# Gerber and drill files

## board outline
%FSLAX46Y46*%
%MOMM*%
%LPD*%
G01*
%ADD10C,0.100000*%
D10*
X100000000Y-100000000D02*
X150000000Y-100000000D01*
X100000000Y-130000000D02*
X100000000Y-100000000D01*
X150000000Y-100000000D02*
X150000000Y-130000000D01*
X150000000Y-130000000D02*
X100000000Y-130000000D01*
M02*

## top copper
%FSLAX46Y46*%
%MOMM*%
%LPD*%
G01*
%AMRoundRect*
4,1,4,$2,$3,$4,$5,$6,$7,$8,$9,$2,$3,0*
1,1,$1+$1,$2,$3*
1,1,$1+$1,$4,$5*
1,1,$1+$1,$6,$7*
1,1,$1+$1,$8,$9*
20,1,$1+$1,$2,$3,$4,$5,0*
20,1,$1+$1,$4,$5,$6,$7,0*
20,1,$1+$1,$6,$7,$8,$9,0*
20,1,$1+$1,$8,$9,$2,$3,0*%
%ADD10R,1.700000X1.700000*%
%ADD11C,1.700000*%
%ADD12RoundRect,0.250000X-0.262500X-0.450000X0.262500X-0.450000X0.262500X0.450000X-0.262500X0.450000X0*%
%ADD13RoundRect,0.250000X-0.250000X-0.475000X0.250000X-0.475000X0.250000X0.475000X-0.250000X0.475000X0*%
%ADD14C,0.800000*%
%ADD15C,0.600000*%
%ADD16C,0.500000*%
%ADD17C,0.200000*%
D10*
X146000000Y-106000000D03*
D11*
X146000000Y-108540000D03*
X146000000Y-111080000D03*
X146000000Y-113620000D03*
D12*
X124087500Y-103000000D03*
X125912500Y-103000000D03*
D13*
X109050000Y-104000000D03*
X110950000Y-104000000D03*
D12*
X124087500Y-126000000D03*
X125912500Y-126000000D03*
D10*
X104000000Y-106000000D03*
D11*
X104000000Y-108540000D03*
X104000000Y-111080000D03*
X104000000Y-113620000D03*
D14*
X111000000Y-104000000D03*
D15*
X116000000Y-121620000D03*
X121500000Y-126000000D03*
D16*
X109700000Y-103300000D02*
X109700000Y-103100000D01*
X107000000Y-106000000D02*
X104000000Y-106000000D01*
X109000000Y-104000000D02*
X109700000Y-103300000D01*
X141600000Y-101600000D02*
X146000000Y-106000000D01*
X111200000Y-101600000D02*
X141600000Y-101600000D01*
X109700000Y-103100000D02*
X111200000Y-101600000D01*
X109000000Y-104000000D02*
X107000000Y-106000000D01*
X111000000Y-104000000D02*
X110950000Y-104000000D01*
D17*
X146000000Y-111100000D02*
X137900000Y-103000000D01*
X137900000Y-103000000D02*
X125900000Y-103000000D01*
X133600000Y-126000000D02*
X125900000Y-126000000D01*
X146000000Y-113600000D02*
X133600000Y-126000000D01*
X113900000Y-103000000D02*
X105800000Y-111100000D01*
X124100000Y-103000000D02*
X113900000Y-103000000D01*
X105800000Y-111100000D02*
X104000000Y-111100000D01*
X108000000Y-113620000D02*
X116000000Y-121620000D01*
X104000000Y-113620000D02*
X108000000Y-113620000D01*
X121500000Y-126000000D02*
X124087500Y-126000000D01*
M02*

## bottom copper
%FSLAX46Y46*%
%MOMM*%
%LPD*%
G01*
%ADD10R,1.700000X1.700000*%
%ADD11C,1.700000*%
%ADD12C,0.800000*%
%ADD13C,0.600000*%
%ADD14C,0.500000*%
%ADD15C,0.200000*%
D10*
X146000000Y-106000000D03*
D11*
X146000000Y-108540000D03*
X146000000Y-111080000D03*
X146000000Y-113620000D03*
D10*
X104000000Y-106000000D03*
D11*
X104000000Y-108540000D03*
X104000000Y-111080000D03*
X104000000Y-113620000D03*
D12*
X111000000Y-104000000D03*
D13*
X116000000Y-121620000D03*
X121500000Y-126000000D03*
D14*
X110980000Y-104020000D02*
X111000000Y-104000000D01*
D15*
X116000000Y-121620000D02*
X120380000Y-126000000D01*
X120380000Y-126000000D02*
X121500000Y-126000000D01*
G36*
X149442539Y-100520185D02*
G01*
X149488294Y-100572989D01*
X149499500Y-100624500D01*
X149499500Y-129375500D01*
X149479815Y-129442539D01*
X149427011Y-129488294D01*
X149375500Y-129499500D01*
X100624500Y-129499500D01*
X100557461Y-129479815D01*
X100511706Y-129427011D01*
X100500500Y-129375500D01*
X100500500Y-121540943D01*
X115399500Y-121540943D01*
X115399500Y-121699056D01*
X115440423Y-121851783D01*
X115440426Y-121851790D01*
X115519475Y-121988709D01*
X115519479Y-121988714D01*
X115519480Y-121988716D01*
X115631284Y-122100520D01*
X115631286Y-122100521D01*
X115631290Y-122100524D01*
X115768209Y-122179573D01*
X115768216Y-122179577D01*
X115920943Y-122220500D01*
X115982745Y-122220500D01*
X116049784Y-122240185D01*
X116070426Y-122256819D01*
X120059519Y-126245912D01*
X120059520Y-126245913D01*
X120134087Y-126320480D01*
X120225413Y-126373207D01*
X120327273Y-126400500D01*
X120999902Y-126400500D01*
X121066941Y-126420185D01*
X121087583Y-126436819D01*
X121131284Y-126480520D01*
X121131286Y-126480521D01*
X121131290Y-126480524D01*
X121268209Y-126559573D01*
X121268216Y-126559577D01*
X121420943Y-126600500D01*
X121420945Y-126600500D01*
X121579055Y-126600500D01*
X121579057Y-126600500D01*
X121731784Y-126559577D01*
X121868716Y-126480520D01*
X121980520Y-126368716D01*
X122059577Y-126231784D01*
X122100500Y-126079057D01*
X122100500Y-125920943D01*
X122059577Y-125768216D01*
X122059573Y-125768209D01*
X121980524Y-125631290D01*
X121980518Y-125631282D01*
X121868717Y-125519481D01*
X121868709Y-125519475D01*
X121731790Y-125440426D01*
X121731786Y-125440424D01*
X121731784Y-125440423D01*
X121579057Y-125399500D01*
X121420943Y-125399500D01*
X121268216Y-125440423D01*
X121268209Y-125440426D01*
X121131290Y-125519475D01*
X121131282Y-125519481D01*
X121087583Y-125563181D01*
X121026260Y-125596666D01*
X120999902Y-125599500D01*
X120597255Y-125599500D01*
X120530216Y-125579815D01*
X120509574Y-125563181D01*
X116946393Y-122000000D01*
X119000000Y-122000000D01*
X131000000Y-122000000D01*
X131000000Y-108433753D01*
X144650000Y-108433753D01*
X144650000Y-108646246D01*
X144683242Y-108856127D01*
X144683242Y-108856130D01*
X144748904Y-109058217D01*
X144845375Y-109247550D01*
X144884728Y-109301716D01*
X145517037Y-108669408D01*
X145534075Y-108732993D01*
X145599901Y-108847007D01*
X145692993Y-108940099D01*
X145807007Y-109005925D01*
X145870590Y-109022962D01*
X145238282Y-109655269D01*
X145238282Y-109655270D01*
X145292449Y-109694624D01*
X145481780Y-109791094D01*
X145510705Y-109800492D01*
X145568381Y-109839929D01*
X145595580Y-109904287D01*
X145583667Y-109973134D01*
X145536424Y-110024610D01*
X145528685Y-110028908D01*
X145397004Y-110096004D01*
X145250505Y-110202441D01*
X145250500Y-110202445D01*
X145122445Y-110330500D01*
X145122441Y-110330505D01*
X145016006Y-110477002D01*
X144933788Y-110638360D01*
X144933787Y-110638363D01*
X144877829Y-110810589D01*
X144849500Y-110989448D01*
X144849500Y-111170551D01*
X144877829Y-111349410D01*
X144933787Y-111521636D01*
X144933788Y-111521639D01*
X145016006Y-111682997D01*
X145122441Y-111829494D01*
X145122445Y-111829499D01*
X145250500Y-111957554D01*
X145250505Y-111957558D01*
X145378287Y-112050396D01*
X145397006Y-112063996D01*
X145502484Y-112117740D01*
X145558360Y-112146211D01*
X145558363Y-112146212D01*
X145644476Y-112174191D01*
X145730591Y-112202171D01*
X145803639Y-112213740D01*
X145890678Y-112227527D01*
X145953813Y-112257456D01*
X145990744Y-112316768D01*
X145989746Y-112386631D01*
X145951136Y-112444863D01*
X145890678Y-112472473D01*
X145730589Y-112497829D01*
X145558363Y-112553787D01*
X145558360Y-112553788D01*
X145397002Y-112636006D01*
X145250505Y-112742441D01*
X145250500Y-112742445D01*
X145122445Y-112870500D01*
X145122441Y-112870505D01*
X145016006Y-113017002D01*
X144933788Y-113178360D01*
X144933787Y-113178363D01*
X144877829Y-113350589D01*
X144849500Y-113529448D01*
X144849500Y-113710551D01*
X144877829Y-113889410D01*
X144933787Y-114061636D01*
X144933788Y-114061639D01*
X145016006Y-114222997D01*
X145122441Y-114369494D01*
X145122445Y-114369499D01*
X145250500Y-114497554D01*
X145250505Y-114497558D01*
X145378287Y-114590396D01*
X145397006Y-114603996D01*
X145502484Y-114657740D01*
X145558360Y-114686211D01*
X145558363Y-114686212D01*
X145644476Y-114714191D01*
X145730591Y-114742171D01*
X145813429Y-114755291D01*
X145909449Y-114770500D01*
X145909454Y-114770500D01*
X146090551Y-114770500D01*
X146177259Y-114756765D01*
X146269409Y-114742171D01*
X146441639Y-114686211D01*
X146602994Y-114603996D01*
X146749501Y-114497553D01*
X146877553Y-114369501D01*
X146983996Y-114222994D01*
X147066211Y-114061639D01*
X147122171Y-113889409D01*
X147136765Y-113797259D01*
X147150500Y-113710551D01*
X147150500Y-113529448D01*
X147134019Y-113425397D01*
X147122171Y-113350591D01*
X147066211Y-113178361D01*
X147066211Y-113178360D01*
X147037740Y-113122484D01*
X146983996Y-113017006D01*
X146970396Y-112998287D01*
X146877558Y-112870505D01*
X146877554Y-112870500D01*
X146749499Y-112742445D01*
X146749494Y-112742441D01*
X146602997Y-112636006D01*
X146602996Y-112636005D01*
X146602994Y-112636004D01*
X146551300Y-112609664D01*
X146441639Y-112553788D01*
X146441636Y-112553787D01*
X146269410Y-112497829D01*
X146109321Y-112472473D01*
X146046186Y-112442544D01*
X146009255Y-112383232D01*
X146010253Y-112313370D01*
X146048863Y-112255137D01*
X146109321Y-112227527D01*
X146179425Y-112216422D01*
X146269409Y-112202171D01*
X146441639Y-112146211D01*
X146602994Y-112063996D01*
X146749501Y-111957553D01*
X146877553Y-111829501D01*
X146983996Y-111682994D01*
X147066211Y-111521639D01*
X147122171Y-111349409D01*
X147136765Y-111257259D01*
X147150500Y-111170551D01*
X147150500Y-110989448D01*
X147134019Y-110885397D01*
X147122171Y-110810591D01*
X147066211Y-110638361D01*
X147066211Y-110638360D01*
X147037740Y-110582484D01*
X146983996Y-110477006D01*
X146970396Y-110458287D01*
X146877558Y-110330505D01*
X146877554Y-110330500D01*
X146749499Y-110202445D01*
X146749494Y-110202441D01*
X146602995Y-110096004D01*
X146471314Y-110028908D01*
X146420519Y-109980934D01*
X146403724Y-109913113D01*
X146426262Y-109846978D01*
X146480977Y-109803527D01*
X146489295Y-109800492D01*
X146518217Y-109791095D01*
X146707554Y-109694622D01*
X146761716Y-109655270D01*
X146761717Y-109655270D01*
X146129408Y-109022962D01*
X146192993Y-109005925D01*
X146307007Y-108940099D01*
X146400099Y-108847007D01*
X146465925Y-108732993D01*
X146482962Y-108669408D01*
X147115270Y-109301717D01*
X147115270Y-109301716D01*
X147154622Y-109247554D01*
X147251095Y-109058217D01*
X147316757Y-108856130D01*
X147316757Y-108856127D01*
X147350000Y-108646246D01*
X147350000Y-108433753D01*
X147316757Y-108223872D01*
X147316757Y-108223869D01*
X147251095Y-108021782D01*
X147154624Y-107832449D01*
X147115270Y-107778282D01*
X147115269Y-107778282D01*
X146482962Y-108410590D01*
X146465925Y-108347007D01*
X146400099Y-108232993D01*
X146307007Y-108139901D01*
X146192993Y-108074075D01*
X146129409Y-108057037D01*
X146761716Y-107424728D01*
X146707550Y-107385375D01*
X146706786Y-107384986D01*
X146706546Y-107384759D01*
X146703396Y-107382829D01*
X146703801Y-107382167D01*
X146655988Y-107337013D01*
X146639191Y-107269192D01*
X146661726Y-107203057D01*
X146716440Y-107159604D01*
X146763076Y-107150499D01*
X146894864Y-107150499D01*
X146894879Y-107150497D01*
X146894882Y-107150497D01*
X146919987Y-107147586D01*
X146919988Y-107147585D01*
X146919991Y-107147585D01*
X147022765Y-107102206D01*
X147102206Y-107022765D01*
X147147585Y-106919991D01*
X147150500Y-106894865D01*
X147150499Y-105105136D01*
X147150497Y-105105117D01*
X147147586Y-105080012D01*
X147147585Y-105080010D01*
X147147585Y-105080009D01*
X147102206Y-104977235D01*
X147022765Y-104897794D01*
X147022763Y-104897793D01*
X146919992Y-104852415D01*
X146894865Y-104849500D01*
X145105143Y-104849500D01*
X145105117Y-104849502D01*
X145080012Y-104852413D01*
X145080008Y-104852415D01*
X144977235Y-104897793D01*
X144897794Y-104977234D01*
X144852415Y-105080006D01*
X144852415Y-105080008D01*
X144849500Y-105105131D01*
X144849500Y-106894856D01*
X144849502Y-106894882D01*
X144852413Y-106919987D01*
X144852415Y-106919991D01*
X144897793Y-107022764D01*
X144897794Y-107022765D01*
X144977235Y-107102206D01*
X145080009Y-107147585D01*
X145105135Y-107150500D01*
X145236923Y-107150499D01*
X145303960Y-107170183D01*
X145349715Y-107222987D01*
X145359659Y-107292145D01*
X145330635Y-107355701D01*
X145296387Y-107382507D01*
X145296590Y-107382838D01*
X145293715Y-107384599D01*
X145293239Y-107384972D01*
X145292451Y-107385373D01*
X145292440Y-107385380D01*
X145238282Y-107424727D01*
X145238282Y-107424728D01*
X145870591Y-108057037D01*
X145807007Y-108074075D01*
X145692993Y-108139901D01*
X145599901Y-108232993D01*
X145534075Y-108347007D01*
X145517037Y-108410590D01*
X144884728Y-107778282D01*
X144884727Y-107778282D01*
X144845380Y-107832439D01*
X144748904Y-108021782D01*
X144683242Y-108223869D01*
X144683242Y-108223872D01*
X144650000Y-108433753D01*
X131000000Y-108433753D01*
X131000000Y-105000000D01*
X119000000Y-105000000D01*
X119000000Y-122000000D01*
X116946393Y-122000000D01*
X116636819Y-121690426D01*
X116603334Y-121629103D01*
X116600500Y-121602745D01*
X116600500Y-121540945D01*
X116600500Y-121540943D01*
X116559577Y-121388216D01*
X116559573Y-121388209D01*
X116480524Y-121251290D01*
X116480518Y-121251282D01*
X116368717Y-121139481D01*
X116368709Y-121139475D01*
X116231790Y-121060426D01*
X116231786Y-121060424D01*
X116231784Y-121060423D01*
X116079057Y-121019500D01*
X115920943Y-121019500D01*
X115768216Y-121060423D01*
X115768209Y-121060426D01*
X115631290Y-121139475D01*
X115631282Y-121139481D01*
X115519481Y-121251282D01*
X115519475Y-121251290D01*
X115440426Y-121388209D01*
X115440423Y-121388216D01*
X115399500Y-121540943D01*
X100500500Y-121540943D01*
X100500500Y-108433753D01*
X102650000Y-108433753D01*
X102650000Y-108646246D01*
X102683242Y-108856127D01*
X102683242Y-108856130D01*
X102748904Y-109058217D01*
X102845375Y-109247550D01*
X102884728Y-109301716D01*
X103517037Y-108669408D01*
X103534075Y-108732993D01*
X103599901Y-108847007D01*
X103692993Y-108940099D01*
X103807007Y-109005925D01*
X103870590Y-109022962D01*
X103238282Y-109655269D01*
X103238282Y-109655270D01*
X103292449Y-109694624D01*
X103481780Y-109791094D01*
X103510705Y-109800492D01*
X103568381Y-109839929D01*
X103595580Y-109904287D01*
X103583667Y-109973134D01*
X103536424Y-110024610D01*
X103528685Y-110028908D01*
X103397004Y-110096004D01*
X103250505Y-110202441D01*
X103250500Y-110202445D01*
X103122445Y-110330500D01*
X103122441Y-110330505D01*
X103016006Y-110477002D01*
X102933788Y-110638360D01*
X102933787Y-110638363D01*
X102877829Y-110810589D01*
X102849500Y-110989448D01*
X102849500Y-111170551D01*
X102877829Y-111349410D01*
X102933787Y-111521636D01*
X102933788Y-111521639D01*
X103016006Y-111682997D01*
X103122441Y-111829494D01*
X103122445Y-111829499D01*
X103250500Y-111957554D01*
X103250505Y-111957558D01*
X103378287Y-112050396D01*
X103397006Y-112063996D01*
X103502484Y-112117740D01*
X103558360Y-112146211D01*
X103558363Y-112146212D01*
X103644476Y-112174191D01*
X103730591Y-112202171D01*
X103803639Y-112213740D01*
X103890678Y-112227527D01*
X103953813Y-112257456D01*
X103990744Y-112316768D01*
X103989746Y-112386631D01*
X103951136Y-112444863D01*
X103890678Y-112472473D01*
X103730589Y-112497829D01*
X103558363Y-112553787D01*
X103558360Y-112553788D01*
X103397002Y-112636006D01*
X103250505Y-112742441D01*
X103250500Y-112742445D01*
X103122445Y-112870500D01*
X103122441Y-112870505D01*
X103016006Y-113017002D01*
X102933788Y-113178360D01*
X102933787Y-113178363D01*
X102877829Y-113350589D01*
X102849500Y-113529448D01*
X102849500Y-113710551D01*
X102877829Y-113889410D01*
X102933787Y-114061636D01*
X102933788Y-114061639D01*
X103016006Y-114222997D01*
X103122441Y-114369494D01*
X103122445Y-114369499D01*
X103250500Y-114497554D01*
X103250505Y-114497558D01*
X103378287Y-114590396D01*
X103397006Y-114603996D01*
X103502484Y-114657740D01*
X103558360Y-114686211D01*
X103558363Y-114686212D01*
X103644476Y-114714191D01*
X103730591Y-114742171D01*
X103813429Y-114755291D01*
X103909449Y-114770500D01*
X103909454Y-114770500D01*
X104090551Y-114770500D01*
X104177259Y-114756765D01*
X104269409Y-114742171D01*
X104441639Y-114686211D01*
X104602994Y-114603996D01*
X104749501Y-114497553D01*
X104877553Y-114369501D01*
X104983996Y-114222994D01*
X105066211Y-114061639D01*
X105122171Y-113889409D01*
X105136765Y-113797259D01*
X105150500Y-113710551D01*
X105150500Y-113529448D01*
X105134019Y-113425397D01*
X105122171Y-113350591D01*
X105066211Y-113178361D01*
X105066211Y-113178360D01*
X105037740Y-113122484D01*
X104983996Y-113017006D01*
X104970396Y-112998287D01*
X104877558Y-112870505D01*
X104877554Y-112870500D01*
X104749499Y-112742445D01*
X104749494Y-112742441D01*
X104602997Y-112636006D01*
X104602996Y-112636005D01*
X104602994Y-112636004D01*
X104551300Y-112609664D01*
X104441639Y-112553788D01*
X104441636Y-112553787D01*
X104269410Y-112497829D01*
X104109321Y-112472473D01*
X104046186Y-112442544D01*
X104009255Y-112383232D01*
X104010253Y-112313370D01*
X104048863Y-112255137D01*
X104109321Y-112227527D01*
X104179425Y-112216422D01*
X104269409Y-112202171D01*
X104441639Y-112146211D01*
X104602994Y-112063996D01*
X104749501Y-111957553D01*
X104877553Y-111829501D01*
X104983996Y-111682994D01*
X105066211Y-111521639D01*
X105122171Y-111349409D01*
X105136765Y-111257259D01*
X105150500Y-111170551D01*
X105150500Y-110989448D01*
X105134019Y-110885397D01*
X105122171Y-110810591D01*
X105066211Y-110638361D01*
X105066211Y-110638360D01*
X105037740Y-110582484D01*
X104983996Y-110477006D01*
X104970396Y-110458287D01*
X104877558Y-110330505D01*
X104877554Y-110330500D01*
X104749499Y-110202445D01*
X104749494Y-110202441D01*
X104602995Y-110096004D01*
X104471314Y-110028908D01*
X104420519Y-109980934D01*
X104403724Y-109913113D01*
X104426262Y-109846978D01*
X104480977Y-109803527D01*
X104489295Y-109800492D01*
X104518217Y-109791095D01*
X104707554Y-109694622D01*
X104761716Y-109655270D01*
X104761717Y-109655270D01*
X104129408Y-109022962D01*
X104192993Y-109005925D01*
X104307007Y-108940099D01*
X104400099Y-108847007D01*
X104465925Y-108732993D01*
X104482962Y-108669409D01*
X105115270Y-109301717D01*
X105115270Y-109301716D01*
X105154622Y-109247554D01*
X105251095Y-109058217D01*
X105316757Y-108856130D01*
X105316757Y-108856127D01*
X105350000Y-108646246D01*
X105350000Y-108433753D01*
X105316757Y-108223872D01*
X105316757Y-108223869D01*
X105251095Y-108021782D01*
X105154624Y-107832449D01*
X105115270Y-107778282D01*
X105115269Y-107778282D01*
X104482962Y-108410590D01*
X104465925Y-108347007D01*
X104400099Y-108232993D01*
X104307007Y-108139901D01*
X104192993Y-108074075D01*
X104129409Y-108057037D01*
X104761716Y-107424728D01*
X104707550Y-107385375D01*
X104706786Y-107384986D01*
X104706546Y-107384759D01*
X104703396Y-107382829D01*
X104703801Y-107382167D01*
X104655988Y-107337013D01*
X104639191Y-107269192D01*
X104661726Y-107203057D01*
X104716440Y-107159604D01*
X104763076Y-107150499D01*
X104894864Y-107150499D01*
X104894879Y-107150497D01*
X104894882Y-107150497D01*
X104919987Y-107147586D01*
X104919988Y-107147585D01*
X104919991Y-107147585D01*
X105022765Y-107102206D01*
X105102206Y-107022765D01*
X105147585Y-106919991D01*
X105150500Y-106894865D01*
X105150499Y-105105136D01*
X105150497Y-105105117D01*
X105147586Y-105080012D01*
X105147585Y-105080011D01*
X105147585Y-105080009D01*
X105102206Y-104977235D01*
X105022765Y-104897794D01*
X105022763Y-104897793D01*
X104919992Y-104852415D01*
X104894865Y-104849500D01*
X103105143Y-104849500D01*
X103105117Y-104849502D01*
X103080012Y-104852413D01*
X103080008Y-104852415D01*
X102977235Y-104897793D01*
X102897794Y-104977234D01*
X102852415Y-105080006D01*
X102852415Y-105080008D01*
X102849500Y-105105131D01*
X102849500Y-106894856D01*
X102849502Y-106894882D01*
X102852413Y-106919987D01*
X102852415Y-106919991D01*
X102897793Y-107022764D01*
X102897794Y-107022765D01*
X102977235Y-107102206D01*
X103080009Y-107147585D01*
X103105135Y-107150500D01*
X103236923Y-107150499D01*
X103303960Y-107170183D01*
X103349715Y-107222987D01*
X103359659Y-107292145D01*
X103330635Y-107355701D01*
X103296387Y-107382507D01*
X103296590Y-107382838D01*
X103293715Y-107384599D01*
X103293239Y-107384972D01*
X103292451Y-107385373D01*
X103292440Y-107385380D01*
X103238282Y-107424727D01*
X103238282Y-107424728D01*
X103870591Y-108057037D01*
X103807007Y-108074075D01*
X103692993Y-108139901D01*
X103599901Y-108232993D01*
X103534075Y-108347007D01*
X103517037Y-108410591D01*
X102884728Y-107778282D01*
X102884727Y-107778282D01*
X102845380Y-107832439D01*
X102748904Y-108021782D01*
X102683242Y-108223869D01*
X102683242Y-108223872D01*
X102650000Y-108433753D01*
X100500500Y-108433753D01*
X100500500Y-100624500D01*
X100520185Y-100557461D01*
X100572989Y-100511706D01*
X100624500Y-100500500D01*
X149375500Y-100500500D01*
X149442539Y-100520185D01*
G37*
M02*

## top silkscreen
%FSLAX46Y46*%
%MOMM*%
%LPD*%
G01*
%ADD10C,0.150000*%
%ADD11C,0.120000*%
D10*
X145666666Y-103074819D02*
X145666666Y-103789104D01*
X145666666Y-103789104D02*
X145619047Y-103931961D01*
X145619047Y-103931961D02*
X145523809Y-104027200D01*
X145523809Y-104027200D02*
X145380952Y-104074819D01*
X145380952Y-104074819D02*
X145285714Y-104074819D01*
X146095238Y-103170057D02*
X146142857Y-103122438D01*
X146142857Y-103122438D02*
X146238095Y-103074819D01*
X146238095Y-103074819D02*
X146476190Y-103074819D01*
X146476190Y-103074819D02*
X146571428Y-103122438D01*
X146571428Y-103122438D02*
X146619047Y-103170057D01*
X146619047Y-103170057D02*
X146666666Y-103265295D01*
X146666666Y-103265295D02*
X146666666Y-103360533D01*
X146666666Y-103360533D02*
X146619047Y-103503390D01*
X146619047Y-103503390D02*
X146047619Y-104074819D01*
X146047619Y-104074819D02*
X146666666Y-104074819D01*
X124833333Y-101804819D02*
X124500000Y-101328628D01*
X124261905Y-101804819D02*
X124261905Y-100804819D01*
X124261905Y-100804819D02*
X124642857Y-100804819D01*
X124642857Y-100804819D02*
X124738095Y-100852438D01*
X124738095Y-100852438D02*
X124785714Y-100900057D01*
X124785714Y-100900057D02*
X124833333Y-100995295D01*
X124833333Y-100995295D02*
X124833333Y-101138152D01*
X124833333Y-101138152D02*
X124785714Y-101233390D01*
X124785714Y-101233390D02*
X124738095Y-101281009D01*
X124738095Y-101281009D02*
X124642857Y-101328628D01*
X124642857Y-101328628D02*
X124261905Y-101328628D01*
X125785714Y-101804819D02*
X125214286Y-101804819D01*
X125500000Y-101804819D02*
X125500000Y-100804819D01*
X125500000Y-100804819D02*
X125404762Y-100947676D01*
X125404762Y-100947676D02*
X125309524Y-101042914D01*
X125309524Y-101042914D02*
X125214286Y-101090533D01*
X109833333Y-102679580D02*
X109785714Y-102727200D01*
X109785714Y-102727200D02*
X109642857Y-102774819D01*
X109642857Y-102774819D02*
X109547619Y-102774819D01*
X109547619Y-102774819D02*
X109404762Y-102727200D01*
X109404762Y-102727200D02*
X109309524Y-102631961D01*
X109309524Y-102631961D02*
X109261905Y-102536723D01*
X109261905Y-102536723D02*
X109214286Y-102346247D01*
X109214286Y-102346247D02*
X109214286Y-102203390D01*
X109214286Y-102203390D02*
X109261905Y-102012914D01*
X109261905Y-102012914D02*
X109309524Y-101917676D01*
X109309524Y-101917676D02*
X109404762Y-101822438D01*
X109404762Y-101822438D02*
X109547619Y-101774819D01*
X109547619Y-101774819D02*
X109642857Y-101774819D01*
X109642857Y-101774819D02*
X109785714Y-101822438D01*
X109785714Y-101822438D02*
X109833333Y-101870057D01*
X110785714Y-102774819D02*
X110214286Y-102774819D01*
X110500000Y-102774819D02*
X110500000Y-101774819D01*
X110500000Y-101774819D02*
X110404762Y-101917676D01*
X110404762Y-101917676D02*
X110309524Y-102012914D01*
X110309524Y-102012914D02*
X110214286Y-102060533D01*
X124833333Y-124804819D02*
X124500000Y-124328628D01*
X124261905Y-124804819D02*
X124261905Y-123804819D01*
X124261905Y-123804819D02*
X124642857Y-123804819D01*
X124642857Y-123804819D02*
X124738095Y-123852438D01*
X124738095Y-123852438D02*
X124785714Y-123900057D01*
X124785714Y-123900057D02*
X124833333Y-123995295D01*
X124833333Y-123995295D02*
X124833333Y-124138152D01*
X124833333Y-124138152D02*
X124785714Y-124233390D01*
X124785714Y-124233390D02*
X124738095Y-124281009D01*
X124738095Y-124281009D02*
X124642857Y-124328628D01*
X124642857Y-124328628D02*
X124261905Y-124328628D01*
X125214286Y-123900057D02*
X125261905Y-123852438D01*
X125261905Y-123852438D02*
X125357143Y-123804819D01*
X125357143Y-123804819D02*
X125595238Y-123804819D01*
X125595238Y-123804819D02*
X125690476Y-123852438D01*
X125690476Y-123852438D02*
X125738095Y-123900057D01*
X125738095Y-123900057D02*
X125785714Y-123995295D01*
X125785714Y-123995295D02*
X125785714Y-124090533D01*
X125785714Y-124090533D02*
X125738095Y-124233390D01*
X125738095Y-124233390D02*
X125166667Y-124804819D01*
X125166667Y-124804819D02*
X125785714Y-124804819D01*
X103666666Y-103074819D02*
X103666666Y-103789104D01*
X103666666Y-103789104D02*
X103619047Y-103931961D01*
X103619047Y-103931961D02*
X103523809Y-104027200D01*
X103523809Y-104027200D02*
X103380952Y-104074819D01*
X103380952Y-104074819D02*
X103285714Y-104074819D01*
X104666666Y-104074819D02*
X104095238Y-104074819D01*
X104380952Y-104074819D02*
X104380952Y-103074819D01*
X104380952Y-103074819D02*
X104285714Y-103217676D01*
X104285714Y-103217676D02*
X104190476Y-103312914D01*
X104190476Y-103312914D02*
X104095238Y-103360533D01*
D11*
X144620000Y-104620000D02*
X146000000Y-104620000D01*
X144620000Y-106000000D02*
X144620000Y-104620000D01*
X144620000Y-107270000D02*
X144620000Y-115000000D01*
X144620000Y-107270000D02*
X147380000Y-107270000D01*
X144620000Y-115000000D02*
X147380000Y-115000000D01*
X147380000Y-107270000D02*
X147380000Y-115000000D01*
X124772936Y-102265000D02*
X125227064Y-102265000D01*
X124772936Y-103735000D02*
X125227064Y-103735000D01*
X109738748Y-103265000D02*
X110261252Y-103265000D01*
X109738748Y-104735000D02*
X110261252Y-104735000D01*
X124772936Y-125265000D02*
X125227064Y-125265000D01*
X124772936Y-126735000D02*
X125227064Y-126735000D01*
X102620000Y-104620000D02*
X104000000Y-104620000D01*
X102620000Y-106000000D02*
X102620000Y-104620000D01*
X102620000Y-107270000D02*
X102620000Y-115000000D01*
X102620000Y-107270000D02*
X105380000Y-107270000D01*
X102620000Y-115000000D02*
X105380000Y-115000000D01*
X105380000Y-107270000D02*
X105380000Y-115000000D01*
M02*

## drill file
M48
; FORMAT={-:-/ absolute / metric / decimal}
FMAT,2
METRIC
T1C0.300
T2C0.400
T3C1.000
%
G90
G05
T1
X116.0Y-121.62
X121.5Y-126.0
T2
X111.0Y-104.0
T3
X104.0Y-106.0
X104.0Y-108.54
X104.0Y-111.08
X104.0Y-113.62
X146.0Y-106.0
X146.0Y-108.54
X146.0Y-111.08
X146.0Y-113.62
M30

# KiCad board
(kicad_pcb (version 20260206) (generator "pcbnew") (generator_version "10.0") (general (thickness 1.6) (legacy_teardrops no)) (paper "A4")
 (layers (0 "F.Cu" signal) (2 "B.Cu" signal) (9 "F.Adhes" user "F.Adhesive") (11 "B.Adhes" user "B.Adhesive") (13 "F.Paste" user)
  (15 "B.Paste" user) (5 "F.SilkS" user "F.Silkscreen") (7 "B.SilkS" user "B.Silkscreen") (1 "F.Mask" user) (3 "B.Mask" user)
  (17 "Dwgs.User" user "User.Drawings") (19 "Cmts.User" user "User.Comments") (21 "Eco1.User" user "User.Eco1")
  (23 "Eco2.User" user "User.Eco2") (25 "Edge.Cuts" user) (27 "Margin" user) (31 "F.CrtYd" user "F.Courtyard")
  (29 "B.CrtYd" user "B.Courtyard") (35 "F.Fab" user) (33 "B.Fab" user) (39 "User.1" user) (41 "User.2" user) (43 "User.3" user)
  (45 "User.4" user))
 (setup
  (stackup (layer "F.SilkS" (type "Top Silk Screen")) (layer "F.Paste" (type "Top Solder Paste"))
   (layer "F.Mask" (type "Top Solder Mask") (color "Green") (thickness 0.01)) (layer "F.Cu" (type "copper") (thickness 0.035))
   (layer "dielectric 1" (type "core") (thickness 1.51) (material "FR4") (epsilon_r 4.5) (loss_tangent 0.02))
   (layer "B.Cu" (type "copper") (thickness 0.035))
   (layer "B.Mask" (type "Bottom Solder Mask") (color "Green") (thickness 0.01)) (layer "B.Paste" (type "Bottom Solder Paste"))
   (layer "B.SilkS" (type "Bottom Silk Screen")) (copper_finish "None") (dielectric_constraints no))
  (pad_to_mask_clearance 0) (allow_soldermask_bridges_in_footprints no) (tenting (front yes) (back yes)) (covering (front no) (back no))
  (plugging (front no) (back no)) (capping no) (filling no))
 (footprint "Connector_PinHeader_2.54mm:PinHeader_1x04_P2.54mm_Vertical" (layer "F.Cu") (at 146 106)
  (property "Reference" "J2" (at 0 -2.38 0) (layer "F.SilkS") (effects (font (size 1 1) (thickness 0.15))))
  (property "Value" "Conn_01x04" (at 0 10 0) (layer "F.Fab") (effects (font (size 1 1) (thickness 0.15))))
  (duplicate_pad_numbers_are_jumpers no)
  (fp_line (start -1.38 -1.38) (end 0 -1.38) (stroke (width 0.12) (type solid)) (layer "F.SilkS"))
  (fp_line (start -1.38 0) (end -1.38 -1.38) (stroke (width 0.12) (type solid)) (layer "F.SilkS"))
  (fp_line (start -1.38 1.27) (end -1.38 9) (stroke (width 0.12) (type solid)) (layer "F.SilkS"))
  (fp_line (start -1.38 1.27) (end 1.38 1.27) (stroke (width 0.12) (type solid)) (layer "F.SilkS"))
  (fp_line (start -1.38 9) (end 1.38 9) (stroke (width 0.12) (type solid)) (layer "F.SilkS"))
  (fp_line (start 1.38 1.27) (end 1.38 9) (stroke (width 0.12) (type solid)) (layer "F.SilkS"))
  (pad "1" thru_hole rect (at 0 0) (size 1.7 1.7) (drill 1) (layers "*.Cu" "*.Mask") (remove_unused_layers no) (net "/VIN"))
  (pad "2" thru_hole circle (at 0 2.54) (size 1.7 1.7) (drill 1) (layers "*.Cu" "*.Mask") (remove_unused_layers no) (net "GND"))
  (pad "3" thru_hole circle (at 0 5.08) (size 1.7 1.7) (drill 1) (layers "*.Cu" "*.Mask") (remove_unused_layers no) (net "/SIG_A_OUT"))
  (pad "4" thru_hole circle (at 0 7.62) (size 1.7 1.7) (drill 1) (layers "*.Cu" "*.Mask") (remove_unused_layers no) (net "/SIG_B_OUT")))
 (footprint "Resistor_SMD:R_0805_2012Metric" (layer "F.Cu") (at 125 103)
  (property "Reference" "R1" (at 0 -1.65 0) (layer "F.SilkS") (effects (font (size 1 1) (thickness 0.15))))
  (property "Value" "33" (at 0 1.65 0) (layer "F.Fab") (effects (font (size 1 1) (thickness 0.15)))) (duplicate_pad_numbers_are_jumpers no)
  (fp_line (start -0.227064 -0.735) (end 0.227064 -0.735) (stroke (width 0.12) (type solid)) (layer "F.SilkS"))
  (fp_line (start -0.227064 0.735) (end 0.227064 0.735) (stroke (width 0.12) (type solid)) (layer "F.SilkS"))
  (pad "1" smd roundrect (at -0.9125 0) (size 1.025 1.4) (layers "F.Cu" "F.Mask" "F.Paste") (roundrect_rratio 0.243902) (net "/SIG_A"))
  (pad "2" smd roundrect (at 0.9125 0) (size 1.025 1.4) (layers "F.Cu" "F.Mask" "F.Paste") (roundrect_rratio 0.243902) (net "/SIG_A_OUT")))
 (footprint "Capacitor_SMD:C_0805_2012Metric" (layer "F.Cu") (at 110 104)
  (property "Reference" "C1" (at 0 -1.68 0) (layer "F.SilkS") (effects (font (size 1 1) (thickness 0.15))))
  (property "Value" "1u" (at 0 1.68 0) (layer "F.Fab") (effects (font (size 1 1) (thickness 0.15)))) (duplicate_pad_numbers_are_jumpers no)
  (fp_line (start -0.261252 -0.735) (end 0.261252 -0.735) (stroke (width 0.12) (type solid)) (layer "F.SilkS"))
  (fp_line (start -0.261252 0.735) (end 0.261252 0.735) (stroke (width 0.12) (type solid)) (layer "F.SilkS"))
  (pad "1" smd roundrect (at -0.95 0) (size 1 1.45) (layers "F.Cu" "F.Mask" "F.Paste") (roundrect_rratio 0.25) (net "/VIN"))
  (pad "2" smd roundrect (at 0.95 0) (size 1 1.45) (layers "F.Cu" "F.Mask" "F.Paste") (roundrect_rratio 0.25) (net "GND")))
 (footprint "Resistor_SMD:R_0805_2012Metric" (layer "F.Cu") (at 125 126)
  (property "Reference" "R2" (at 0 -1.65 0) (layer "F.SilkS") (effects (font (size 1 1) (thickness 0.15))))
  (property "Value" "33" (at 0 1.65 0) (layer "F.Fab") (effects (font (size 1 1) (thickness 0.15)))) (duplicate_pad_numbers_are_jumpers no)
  (fp_line (start -0.227064 -0.735) (end 0.227064 -0.735) (stroke (width 0.12) (type solid)) (layer "F.SilkS"))
  (fp_line (start -0.227064 0.735) (end 0.227064 0.735) (stroke (width 0.12) (type solid)) (layer "F.SilkS"))
  (pad "1" smd roundrect (at -0.9125 0) (size 1.025 1.4) (layers "F.Cu" "F.Mask" "F.Paste") (roundrect_rratio 0.243902) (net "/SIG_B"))
  (pad "2" smd roundrect (at 0.9125 0) (size 1.025 1.4) (layers "F.Cu" "F.Mask" "F.Paste") (roundrect_rratio 0.243902) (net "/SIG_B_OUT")))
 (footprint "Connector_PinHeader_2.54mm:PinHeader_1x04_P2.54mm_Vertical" (layer "F.Cu") (at 104 106)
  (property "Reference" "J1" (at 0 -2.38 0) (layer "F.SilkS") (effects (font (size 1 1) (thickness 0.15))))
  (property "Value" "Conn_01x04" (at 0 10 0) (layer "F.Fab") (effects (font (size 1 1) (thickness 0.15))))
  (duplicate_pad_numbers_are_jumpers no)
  (fp_line (start -1.38 -1.38) (end 0 -1.38) (stroke (width 0.12) (type solid)) (layer "F.SilkS"))
  (fp_line (start -1.38 0) (end -1.38 -1.38) (stroke (width 0.12) (type solid)) (layer "F.SilkS"))
  (fp_line (start -1.38 1.27) (end -1.38 9) (stroke (width 0.12) (type solid)) (layer "F.SilkS"))
  (fp_line (start -1.38 1.27) (end 1.38 1.27) (stroke (width 0.12) (type solid)) (layer "F.SilkS"))
  (fp_line (start -1.38 9) (end 1.38 9) (stroke (width 0.12) (type solid)) (layer "F.SilkS"))
  (fp_line (start 1.38 1.27) (end 1.38 9) (stroke (width 0.12) (type solid)) (layer "F.SilkS"))
  (pad "1" thru_hole rect (at 0 0) (size 1.7 1.7) (drill 1) (layers "*.Cu" "*.Mask") (remove_unused_layers no) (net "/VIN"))
  (pad "2" thru_hole circle (at 0 2.54) (size 1.7 1.7) (drill 1) (layers "*.Cu" "*.Mask") (remove_unused_layers no) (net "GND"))
  (pad "3" thru_hole circle (at 0 5.08) (size 1.7 1.7) (drill 1) (layers "*.Cu" "*.Mask") (remove_unused_layers no) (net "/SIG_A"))
  (pad "4" thru_hole circle (at 0 7.62) (size 1.7 1.7) (drill 1) (layers "*.Cu" "*.Mask") (remove_unused_layers no) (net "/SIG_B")))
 (gr_line (start 100 100) (end 150 100) (stroke (width 0.1) (type default)) (layer "Edge.Cuts"))
 (gr_line (start 100 130) (end 100 100) (stroke (width 0.1) (type default)) (layer "Edge.Cuts"))
 (gr_line (start 150 100) (end 150 130) (stroke (width 0.1) (type default)) (layer "Edge.Cuts"))
 (gr_line (start 150 130) (end 100 130) (stroke (width 0.1) (type default)) (layer "Edge.Cuts"))
 (segment (start 109.7 103.3) (end 109.7 103.1) (width 0.5) (layer "F.Cu") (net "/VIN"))
 (segment (start 107 106) (end 104 106) (width 0.5) (layer "F.Cu") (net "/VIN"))
 (segment (start 109 104) (end 109.7 103.3) (width 0.5) (layer "F.Cu") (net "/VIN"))
 (segment (start 141.6 101.6) (end 146 106) (width 0.5) (layer "F.Cu") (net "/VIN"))
 (segment (start 111.2 101.6) (end 141.6 101.6) (width 0.5) (layer "F.Cu") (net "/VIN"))
 (segment (start 109.7 103.1) (end 111.2 101.6) (width 0.5) (layer "F.Cu") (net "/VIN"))
 (segment (start 109 104) (end 107 106) (width 0.5) (layer "F.Cu") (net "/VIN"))
 (segment (start 111 104) (end 110.95 104) (width 0.5) (layer "F.Cu") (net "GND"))
 (via (at 111 104) (size 0.8) (drill 0.4) (layers "F.Cu" "B.Cu") (capping yes) (filling yes) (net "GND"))
 (segment (start 110.98 104.02) (end 111 104) (width 0.5) (layer "B.Cu") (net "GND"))
 (segment (start 146 111.1) (end 137.9 103) (width 0.2) (layer "F.Cu") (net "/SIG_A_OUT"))
 (segment (start 137.9 103) (end 125.9 103) (width 0.2) (layer "F.Cu") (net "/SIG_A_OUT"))
 (segment (start 133.6 126) (end 125.9 126) (width 0.2) (layer "F.Cu") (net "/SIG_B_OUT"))
 (segment (start 146 113.6) (end 133.6 126) (width 0.2) (layer "F.Cu") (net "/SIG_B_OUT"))
 (segment (start 113.9 103) (end 105.8 111.1) (width 0.2) (layer "F.Cu") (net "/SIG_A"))
 (segment (start 124.1 103) (end 113.9 103) (width 0.2) (layer "F.Cu") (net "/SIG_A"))
 (segment (start 105.8 111.1) (end 104 111.1) (width 0.2) (layer "F.Cu") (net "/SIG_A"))
 (segment (start 108 113.62) (end 116 121.62) (width 0.2) (locked yes) (layer "F.Cu") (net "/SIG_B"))
 (segment (start 104 113.62) (end 108 113.62) (width 0.2) (locked yes) (layer "F.Cu") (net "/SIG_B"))
 (segment (start 121.5 126) (end 124.0875 126) (width 0.2) (locked yes) (layer "F.Cu") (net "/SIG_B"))
 (via (at 116 121.62) (size 0.6) (drill 0.3) (layers "F.Cu" "B.Cu") (locked yes) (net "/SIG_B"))
 (via (at 121.5 126) (size 0.6) (drill 0.3) (layers "F.Cu" "B.Cu") (locked yes) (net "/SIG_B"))
 (segment (start 116 121.62) (end 120.38 126) (width 0.2) (locked yes) (layer "B.Cu") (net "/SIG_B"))
 (segment (start 120.38 126) (end 121.5 126) (width 0.2) (locked yes) (layer "B.Cu") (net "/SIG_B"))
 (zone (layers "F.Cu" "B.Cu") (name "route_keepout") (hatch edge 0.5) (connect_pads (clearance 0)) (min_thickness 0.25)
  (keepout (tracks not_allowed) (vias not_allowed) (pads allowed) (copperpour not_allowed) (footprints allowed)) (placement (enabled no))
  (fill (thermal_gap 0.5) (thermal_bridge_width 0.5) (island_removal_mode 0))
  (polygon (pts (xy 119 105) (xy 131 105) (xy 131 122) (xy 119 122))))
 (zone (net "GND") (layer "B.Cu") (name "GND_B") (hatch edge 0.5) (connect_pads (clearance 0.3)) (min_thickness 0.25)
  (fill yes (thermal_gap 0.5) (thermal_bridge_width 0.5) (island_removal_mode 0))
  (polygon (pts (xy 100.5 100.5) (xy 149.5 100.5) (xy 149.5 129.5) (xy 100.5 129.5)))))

